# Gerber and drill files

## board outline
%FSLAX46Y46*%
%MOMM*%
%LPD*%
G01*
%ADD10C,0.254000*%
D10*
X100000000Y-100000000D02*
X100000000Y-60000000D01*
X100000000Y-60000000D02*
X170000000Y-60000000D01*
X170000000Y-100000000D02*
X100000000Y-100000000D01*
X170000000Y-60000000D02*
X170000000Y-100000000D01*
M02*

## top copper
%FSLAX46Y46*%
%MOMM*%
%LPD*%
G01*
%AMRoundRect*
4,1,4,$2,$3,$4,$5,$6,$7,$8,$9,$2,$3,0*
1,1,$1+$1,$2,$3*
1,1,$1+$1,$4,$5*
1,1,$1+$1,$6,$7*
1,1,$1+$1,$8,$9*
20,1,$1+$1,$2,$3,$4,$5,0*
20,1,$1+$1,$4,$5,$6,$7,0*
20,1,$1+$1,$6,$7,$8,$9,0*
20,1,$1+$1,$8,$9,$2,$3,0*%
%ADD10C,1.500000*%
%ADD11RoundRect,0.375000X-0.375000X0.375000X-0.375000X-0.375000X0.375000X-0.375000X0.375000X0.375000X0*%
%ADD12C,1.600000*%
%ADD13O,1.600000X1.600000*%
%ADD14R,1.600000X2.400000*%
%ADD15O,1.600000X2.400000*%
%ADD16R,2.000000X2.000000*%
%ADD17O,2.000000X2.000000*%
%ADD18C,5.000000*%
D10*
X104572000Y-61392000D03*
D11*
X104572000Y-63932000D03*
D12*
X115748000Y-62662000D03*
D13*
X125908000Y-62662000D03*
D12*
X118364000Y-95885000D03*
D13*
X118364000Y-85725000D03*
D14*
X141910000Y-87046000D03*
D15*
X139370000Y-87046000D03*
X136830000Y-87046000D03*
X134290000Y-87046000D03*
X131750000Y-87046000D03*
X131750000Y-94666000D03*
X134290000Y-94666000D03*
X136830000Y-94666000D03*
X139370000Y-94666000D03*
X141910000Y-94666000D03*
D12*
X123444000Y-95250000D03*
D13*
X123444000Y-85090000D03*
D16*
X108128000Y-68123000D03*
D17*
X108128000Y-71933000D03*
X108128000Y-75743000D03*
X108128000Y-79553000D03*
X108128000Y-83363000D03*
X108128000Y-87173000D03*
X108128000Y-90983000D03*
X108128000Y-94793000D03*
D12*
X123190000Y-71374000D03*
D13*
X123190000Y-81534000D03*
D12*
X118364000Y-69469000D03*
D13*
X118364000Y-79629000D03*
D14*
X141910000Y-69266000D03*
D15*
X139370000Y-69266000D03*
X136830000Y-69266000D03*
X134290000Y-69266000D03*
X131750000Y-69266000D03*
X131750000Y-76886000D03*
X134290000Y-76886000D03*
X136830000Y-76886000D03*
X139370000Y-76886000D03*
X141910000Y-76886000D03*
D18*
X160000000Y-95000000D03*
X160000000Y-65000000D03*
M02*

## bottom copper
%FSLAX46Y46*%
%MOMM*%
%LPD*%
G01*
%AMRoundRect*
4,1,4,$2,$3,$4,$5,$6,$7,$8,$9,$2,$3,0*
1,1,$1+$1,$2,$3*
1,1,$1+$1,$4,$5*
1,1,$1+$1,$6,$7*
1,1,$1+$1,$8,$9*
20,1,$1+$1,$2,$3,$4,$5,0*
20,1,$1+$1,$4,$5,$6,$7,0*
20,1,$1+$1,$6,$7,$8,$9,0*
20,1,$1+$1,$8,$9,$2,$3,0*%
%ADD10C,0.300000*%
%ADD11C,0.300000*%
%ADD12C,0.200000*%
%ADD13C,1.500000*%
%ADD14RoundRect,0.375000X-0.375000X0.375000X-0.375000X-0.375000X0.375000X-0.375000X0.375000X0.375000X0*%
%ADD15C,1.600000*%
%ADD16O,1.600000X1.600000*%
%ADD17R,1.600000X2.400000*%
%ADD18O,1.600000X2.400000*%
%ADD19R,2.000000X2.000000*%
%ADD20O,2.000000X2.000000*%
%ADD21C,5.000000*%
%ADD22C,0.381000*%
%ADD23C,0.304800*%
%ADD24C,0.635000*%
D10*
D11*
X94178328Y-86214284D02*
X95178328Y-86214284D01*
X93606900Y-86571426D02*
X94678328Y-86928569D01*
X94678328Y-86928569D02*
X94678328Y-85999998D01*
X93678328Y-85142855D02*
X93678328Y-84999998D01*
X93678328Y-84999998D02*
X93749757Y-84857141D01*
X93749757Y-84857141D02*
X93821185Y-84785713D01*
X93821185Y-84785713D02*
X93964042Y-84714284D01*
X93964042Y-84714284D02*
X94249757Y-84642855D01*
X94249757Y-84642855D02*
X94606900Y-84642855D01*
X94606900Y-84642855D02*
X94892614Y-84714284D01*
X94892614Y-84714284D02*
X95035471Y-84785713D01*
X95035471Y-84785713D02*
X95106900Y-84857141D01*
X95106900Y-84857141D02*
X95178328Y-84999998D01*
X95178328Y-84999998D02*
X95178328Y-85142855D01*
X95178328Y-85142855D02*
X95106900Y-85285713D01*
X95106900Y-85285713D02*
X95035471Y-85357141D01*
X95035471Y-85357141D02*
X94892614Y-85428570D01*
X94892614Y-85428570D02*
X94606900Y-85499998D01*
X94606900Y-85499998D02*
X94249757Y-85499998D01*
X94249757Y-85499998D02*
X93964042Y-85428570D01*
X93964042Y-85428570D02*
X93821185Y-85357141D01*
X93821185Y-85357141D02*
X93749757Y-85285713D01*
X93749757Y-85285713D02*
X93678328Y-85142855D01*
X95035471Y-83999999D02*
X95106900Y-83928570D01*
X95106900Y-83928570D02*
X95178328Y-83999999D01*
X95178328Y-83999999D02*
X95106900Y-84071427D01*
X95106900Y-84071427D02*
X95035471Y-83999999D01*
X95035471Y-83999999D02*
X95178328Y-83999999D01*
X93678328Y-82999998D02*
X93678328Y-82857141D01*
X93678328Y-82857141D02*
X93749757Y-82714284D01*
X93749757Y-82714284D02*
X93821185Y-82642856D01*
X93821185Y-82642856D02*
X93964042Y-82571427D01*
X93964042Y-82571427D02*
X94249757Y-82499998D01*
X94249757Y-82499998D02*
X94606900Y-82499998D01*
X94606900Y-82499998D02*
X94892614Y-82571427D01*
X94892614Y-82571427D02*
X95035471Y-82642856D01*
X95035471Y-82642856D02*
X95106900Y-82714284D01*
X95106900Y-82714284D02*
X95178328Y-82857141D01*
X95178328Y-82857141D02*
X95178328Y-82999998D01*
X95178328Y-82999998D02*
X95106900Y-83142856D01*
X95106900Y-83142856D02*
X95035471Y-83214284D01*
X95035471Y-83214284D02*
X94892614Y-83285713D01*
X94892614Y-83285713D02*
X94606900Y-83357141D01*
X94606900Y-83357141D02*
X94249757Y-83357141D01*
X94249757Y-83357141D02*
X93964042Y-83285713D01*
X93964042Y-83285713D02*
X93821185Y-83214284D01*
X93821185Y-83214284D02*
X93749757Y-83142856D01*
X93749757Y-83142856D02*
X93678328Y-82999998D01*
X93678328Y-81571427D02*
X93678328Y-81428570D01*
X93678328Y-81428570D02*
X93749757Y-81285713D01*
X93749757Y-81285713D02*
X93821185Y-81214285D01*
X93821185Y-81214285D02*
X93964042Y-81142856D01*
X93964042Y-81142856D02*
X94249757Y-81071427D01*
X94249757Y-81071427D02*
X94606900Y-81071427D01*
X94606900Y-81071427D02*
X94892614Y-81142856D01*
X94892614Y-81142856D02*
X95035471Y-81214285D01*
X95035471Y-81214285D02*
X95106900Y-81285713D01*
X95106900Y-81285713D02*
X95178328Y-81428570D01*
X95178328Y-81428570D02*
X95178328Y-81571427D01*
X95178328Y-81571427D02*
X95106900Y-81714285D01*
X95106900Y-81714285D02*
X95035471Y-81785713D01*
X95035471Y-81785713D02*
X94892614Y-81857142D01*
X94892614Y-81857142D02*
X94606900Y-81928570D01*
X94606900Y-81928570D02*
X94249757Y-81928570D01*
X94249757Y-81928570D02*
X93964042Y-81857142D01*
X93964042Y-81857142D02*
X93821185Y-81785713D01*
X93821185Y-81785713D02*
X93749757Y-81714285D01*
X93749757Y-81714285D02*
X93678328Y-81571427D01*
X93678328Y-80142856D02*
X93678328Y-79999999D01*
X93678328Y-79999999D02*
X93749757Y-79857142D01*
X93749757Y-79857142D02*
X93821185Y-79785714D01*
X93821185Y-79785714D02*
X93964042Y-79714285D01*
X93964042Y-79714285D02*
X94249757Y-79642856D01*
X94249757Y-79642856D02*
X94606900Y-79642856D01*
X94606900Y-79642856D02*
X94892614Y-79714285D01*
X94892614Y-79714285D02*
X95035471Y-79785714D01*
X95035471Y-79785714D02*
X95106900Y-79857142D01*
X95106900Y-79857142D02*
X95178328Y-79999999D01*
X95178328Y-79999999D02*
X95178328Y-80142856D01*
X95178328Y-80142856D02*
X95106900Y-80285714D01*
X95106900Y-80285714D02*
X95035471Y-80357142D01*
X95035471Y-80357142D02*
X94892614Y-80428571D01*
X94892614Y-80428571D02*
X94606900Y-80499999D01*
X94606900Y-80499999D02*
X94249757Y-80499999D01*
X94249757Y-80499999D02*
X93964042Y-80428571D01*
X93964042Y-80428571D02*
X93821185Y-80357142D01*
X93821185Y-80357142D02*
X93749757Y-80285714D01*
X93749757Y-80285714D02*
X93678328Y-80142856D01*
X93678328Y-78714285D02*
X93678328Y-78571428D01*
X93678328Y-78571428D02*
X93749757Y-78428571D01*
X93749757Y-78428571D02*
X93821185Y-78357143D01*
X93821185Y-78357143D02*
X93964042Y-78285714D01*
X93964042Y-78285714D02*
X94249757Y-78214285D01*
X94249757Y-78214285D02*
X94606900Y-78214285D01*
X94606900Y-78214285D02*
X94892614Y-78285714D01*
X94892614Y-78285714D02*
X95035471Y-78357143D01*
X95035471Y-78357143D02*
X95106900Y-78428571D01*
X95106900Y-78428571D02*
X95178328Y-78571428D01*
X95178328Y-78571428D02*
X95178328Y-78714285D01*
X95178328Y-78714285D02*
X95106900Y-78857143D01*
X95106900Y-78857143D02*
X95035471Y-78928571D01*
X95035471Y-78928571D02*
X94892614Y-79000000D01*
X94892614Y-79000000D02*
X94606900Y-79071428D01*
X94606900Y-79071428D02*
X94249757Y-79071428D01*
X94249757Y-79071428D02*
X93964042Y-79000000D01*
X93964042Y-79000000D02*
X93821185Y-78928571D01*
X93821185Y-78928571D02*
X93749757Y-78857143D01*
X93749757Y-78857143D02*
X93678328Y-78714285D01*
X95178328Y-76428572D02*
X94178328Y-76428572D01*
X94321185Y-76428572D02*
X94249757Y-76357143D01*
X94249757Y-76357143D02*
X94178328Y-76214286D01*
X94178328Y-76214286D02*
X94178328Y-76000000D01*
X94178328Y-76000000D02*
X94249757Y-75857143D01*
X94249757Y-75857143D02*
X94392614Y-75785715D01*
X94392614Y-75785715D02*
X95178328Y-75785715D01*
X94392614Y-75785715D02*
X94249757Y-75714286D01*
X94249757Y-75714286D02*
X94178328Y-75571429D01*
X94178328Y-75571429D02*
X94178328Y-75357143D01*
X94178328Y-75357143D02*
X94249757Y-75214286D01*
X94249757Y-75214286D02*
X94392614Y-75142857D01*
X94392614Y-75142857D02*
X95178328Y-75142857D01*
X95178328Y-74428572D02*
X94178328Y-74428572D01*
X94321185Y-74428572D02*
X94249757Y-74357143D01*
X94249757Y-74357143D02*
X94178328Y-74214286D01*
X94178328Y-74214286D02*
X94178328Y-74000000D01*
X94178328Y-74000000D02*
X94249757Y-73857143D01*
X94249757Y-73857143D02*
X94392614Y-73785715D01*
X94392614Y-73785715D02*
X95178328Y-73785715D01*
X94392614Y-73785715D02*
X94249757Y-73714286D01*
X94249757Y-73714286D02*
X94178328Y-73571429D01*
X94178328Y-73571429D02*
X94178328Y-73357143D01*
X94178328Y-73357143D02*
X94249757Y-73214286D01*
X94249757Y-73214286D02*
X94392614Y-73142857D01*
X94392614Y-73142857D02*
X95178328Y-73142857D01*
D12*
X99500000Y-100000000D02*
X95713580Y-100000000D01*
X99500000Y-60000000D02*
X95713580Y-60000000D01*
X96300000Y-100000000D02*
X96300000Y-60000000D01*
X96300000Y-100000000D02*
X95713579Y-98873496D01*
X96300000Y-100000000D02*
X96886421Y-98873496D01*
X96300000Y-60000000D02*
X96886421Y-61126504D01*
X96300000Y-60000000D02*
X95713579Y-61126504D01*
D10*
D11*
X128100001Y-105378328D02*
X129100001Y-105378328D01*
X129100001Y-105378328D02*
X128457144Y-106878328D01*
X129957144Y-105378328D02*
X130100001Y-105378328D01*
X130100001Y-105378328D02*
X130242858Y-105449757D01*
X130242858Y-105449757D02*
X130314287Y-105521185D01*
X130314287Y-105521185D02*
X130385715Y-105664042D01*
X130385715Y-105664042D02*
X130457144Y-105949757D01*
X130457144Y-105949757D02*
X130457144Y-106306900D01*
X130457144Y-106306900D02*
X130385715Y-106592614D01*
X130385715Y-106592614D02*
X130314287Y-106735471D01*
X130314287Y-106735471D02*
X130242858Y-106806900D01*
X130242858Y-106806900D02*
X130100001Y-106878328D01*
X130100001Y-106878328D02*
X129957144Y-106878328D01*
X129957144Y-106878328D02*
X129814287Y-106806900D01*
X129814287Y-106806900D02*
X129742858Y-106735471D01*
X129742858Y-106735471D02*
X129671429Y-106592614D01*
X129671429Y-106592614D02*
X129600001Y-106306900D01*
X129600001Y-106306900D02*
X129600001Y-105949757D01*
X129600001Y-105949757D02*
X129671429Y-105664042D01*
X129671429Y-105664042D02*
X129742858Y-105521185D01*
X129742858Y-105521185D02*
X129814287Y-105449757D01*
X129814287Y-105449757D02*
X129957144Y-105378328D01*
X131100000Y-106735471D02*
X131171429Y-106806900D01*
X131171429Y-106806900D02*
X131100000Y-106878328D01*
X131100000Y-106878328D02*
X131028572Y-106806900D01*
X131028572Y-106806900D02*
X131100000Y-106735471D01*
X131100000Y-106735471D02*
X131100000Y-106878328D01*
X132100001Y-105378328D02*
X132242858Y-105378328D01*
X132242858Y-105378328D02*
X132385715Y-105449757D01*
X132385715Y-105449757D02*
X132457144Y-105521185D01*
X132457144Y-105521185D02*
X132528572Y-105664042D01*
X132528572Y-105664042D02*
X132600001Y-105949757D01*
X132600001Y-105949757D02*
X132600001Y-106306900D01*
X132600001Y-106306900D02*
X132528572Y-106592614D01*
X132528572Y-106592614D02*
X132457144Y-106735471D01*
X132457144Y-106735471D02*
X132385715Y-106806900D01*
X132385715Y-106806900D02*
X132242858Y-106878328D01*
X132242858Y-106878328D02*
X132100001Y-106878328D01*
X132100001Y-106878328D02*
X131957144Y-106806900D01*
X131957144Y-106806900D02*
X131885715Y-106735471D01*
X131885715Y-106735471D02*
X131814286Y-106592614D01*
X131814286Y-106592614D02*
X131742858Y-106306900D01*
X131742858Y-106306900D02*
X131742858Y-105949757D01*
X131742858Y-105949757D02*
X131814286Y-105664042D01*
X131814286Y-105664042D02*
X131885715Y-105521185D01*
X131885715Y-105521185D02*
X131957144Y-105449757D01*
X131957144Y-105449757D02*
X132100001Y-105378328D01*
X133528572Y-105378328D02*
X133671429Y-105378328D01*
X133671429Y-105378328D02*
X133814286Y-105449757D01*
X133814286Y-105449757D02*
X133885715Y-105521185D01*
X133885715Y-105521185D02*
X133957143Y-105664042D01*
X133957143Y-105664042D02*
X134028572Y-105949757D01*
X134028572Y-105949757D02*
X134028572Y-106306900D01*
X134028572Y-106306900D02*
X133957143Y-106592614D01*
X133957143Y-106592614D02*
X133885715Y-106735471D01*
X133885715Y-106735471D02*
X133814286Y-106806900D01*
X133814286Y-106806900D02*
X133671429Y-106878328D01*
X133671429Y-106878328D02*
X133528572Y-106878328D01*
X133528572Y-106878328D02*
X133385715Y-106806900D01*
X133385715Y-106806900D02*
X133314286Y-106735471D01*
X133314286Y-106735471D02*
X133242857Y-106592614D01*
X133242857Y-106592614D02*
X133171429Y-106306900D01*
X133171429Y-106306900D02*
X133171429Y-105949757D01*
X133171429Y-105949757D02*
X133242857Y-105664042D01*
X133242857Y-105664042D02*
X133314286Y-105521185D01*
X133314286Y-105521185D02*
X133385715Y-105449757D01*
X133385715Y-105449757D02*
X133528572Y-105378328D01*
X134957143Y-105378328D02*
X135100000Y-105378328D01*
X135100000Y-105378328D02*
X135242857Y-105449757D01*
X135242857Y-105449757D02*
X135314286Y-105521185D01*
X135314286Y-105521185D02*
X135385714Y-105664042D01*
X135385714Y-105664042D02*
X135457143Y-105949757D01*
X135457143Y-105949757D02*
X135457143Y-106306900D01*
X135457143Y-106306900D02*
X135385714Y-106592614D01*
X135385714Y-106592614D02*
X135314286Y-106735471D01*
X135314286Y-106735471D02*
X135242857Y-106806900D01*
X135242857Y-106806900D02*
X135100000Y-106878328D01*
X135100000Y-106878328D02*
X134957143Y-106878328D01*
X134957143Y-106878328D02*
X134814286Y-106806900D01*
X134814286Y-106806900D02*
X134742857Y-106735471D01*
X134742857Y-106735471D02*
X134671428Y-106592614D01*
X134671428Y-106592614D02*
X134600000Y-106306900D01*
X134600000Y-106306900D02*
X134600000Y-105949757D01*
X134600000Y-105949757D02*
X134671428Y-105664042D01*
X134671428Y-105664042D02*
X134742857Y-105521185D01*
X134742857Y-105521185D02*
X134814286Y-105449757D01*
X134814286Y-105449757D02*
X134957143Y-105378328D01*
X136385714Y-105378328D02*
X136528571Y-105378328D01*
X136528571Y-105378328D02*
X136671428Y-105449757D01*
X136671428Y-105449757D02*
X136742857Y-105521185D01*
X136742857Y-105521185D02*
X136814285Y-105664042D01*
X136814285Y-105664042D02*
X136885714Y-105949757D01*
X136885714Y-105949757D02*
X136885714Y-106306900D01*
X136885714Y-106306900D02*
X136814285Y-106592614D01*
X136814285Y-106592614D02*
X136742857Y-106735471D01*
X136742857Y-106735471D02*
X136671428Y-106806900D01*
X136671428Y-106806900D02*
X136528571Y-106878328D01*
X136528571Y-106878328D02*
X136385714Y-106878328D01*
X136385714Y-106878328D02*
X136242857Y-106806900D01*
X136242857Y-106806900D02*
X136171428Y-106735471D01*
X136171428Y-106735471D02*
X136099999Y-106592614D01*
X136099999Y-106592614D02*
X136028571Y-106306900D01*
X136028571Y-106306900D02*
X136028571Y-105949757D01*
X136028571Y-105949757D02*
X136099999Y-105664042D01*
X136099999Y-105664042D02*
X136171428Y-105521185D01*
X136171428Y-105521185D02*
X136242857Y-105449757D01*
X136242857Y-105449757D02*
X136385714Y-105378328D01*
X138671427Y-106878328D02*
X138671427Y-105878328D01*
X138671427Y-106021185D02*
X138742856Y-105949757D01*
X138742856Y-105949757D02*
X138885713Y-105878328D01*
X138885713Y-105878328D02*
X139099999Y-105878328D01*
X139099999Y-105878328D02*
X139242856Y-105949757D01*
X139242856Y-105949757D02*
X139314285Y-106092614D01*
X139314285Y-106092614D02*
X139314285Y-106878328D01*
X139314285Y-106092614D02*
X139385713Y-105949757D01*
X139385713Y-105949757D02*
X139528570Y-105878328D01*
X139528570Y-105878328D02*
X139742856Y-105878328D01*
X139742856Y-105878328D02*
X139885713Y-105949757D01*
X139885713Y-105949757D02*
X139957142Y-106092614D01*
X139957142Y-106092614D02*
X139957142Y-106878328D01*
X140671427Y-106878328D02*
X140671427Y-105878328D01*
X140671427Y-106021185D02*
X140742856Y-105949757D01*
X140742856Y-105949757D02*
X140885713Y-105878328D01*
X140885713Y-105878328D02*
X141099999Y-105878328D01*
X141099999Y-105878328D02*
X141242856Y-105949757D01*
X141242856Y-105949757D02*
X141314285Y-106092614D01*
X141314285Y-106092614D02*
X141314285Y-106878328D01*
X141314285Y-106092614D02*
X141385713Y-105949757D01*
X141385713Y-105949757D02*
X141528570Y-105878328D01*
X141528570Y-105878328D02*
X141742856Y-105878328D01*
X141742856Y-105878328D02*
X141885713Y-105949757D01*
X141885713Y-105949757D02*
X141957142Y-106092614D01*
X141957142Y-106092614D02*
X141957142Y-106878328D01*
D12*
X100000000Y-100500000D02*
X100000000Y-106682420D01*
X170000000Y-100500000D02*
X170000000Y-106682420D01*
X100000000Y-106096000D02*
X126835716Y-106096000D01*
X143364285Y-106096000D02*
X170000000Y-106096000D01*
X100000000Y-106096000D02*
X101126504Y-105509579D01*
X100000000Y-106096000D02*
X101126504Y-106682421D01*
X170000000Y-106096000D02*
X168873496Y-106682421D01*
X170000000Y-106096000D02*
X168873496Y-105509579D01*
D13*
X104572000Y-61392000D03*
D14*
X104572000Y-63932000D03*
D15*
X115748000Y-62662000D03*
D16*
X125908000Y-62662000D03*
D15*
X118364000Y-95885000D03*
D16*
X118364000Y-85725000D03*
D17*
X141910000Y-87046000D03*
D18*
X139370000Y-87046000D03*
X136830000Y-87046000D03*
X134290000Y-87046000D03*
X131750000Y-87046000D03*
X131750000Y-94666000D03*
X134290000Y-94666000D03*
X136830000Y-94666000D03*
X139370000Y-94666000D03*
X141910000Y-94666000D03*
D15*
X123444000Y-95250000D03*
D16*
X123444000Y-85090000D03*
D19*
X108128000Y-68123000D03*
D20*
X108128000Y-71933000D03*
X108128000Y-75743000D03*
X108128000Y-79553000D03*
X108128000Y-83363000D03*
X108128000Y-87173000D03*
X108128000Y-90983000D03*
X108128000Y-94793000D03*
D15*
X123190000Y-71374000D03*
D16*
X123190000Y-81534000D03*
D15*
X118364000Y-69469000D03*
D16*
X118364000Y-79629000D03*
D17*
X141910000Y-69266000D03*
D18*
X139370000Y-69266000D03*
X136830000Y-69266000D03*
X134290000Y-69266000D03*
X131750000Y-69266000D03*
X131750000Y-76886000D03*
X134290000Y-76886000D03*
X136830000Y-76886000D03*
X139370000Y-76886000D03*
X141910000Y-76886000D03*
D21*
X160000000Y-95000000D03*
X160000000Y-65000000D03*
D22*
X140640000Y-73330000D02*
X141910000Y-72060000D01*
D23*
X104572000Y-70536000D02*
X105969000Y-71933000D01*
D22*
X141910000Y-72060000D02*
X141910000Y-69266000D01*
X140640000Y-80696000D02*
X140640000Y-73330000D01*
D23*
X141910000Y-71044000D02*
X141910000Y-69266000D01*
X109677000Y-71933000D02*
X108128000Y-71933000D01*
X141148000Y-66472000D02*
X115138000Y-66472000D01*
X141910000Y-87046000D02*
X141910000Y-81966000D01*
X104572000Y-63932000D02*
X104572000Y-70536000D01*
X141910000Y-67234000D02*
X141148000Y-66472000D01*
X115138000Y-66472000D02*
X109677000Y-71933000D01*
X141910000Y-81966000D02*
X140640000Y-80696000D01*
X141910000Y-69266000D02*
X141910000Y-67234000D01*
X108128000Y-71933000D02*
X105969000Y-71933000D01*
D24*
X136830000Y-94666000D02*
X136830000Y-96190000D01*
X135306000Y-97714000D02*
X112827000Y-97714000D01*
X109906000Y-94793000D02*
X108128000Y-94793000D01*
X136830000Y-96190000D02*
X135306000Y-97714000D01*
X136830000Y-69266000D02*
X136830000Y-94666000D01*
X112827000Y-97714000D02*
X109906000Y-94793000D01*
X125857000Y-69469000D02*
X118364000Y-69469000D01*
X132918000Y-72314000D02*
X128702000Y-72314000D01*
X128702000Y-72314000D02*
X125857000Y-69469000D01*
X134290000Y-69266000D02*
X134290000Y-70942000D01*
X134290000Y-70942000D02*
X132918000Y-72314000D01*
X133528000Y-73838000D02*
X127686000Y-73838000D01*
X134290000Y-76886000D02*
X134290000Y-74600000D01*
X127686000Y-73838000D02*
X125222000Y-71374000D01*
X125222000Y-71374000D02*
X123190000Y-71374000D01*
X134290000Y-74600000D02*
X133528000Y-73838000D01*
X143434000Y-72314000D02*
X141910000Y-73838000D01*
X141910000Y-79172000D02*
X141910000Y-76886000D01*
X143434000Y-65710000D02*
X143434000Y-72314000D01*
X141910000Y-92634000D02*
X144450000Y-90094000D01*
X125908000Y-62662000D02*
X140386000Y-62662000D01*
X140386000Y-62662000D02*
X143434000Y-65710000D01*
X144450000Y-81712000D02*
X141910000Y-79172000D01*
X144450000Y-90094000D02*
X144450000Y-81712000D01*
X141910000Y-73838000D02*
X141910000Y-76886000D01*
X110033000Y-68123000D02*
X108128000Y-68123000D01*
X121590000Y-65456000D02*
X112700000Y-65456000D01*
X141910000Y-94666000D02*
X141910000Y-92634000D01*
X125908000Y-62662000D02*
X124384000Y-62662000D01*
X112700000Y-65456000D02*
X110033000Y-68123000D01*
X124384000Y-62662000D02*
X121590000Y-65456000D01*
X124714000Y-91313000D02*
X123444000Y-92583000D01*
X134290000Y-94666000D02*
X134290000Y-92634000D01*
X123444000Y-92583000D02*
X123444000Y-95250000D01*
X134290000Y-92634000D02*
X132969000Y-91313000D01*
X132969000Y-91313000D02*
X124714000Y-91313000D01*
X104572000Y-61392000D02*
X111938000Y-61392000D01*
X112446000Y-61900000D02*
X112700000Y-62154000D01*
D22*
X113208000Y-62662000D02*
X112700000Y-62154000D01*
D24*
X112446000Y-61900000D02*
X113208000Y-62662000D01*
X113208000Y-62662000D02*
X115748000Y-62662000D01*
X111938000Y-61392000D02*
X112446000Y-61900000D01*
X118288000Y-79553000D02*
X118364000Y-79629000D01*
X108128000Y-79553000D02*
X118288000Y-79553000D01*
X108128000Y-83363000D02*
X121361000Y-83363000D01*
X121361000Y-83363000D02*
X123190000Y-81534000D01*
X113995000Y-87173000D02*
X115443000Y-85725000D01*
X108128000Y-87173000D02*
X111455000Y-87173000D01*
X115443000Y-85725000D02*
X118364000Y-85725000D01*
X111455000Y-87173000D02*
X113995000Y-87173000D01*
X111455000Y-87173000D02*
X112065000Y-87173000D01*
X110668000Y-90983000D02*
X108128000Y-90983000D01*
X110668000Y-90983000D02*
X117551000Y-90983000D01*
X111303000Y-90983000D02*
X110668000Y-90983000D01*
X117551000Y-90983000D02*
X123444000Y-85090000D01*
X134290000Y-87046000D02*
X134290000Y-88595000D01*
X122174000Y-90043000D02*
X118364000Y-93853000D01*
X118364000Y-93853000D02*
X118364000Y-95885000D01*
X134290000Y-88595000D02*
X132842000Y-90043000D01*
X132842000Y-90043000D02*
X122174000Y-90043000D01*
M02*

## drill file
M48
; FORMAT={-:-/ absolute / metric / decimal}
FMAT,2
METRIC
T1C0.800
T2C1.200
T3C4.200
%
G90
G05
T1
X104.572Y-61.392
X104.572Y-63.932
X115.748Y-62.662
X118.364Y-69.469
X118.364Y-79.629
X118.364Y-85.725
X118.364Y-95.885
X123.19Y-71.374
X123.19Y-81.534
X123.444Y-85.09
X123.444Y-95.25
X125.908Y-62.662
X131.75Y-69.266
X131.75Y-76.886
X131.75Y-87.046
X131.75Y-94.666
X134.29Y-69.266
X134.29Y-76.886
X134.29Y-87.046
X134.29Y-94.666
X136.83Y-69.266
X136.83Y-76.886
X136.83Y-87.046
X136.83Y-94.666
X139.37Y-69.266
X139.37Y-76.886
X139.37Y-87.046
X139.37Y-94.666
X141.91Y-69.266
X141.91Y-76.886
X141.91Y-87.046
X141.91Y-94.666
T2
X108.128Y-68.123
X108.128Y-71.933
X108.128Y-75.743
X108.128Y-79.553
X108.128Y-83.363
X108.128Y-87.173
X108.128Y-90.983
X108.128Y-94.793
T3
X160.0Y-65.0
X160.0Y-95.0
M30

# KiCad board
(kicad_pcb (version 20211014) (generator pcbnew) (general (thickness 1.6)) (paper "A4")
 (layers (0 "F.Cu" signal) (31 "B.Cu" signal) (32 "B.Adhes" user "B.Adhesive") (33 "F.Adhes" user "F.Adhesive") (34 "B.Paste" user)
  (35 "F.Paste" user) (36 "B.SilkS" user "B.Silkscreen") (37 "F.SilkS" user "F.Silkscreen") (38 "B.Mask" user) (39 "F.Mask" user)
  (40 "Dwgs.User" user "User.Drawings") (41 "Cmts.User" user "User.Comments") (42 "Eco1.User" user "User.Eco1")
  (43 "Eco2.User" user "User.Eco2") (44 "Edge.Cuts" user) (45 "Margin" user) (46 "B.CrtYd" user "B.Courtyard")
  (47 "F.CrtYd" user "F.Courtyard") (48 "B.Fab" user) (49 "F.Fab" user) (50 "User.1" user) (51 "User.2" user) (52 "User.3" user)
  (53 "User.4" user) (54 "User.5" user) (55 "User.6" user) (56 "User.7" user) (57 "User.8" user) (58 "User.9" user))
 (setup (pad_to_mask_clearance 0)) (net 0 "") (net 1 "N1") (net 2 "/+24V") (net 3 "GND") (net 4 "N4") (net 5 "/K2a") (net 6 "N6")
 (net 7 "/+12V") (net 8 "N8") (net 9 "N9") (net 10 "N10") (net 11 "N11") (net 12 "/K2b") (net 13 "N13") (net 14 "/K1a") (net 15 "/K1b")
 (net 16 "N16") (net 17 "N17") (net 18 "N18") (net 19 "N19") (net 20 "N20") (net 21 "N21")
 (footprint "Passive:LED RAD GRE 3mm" (layer "F.Cu") (at 104.572 62.662 -90)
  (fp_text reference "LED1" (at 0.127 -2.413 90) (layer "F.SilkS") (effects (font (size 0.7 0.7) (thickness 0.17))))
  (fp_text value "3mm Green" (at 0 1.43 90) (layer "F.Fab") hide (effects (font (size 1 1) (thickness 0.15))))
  (pad "1" thru_hole circle (at -1.27 0 270) (size 1.5 1.5) (drill 0.8) (layers *.Cu *.Mask) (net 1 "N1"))
  (pad "2" thru_hole roundrect (at 1.27 0 270) (size 1.5 1.5) (drill 0.8) (layers *.Cu *.Mask) (roundrect_rratio 0.25) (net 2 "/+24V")))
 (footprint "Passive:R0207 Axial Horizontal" (layer "F.Cu") (at 120.828 62.662)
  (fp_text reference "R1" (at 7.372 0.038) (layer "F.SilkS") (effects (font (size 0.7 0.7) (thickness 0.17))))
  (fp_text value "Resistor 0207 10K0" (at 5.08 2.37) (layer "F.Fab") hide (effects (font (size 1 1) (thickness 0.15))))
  (pad "1" thru_hole circle (at -5.08 0) (size 1.6 1.6) (drill 0.8) (layers *.Cu *.Mask) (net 1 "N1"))
  (pad "2" thru_hole oval (at 5.08 0) (size 1.6 1.6) (drill 0.8) (layers *.Cu *.Mask) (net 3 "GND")))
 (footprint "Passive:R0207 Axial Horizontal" (layer "F.Cu") (at 118.364 90.805 90)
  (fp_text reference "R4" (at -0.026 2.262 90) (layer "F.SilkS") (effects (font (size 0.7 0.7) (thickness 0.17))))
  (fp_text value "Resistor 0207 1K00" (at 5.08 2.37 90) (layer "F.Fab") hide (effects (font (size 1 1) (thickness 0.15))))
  (pad "1" thru_hole circle (at -5.08 0 90) (size 1.6 1.6) (drill 0.8) (layers *.Cu *.Mask) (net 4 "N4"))
  (pad "2" thru_hole oval (at 5.08 0 90) (size 1.6 1.6) (drill 0.8) (layers *.Cu *.Mask) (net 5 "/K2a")))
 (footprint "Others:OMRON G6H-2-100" (layer "F.Cu") (at 136.83 90.856 -90)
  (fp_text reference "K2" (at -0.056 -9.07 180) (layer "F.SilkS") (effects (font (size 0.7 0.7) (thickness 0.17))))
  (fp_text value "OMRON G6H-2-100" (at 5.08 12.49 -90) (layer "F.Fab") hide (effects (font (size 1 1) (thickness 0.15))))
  (pad "1" thru_hole rect (at -3.81 -5.08 270) (size 2.4 1.6) (drill 0.8) (layers *.Cu *.Mask) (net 2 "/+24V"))
  (pad "2" thru_hole oval (at -3.81 -2.54 270) (size 2.4 1.6) (drill 0.8) (layers *.Cu *.Mask) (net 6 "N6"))
  (pad "3" thru_hole oval (at -3.81 0 270) (size 2.4 1.6) (drill 0.8) (layers *.Cu *.Mask) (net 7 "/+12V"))
  (pad "4" thru_hole oval (at -3.81 2.54 270) (size 2.4 1.6) (drill 0.8) (layers *.Cu *.Mask) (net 4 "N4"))
  (pad "5" thru_hole oval (at -3.81 5.08 270) (size 2.4 1.6) (drill 0.8) (layers *.Cu *.Mask) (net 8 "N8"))
  (pad "6" thru_hole oval (at 3.81 5.08 270) (size 2.4 1.6) (drill 0.8) (layers *.Cu *.Mask) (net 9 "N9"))
  (pad "7" thru_hole oval (at 3.81 2.54 270) (size 2.4 1.6) (drill 0.8) (layers *.Cu *.Mask) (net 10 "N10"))
  (pad "8" thru_hole oval (at 3.81 0 270) (size 2.4 1.6) (drill 0.8) (layers *.Cu *.Mask) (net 7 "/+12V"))
  (pad "9" thru_hole oval (at 3.81 -2.54 270) (size 2.4 1.6) (drill 0.8) (layers *.Cu *.Mask) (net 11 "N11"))
  (pad "10" thru_hole oval (at 3.81 -5.08 270) (size 2.4 1.6) (drill 0.8) (layers *.Cu *.Mask) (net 3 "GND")))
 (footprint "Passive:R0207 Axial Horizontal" (layer "F.Cu") (at 123.444 90.17 90)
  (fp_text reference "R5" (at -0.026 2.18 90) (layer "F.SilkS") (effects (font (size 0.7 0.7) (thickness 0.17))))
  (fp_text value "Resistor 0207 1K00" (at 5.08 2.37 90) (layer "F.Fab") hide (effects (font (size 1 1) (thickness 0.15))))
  (pad "1" thru_hole circle (at -5.08 0 90) (size 1.6 1.6) (drill 0.8) (layers *.Cu *.Mask) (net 10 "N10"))
  (pad "2" thru_hole oval (at 5.08 0 90) (size 1.6 1.6) (drill 0.8) (layers *.Cu *.Mask) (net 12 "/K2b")))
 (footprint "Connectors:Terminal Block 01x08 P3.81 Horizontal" (layer "F.Cu") (at 108.128 81.458 -90)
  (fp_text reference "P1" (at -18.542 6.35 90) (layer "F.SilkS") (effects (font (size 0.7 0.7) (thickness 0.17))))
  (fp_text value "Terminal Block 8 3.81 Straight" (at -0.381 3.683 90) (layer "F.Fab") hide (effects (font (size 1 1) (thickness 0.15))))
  (pad "1" thru_hole rect (at -13.335 0) (size 2 2) (drill 1.2) (layers *.Cu *.Mask) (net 3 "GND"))
  (pad "2" thru_hole oval (at -9.525 0) (size 2 2) (drill 1.2) (layers *.Cu *.Mask) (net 2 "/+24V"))
  (pad "3" thru_hole oval (at -5.715 0) (size 2 2) (drill 1.2) (layers *.Cu *.Mask) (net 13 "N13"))
  (pad "4" thru_hole oval (at -1.905 0) (size 2 2) (drill 1.2) (layers *.Cu *.Mask) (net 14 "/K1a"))
  (pad "5" thru_hole oval (at 1.905 0) (size 2 2) (drill 1.2) (layers *.Cu *.Mask) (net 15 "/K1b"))
  (pad "6" thru_hole oval (at 5.715 0) (size 2 2) (drill 1.2) (layers *.Cu *.Mask) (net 5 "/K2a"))
  (pad "7" thru_hole oval (at 9.525 0) (size 2 2) (drill 1.2) (layers *.Cu *.Mask) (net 12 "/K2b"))
  (pad "8" thru_hole oval (at 13.335 0) (size 2 2) (drill 1.2) (layers *.Cu *.Mask) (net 7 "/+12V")))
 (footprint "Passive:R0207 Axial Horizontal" (layer "F.Cu") (at 123.19 76.454 -90)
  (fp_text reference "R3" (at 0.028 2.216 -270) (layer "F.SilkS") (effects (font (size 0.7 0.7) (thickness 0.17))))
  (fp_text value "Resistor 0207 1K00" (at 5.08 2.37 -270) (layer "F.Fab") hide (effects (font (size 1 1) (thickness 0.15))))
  (pad "1" thru_hole circle (at -5.08 0 270) (size 1.6 1.6) (drill 0.8) (layers *.Cu *.Mask) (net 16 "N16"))
  (pad "2" thru_hole oval (at 5.08 0 270) (size 1.6 1.6) (drill 0.8) (layers *.Cu *.Mask) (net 15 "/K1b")))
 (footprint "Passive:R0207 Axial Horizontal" (layer "F.Cu") (at 118.364 74.549 -90)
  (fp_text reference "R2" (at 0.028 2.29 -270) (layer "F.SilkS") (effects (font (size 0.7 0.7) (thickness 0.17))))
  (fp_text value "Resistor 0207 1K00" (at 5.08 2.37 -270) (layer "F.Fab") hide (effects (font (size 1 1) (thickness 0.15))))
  (pad "1" thru_hole circle (at -5.08 0 270) (size 1.6 1.6) (drill 0.8) (layers *.Cu *.Mask) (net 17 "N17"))
  (pad "2" thru_hole oval (at 5.08 0 270) (size 1.6 1.6) (drill 0.8) (layers *.Cu *.Mask) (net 14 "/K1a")))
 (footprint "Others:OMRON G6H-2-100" (layer "F.Cu") (at 136.83 73.076 -90)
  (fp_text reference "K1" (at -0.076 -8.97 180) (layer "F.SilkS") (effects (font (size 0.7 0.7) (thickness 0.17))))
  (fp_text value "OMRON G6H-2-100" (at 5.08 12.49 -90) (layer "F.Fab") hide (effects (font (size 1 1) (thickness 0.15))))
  (pad "1" thru_hole rect (at -3.81 -5.08 270) (size 2.4 1.6) (drill 0.8) (layers *.Cu *.Mask) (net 2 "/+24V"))
  (pad "2" thru_hole oval (at -3.81 -2.54 270) (size 2.4 1.6) (drill 0.8) (layers *.Cu *.Mask) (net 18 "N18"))
  (pad "3" thru_hole oval (at -3.81 0 270) (size 2.4 1.6) (drill 0.8) (layers *.Cu *.Mask) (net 7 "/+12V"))
  (pad "4" thru_hole oval (at -3.81 2.54 270) (size 2.4 1.6) (drill 0.8) (layers *.Cu *.Mask) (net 17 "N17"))
  (pad "5" thru_hole oval (at -3.81 5.08 270) (size 2.4 1.6) (drill 0.8) (layers *.Cu *.Mask) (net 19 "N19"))
  (pad "6" thru_hole oval (at 3.81 5.08 270) (size 2.4 1.6) (drill 0.8) (layers *.Cu *.Mask) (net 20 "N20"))
  (pad "7" thru_hole oval (at 3.81 2.54 270) (size 2.4 1.6) (drill 0.8) (layers *.Cu *.Mask) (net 16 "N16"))
  (pad "8" thru_hole oval (at 3.81 0 270) (size 2.4 1.6) (drill 0.8) (layers *.Cu *.Mask) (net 7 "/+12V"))
  (pad "9" thru_hole oval (at 3.81 -2.54 270) (size 2.4 1.6) (drill 0.8) (layers *.Cu *.Mask) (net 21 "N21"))
  (pad "10" thru_hole oval (at 3.81 -5.08 270) (size 2.4 1.6) (drill 0.8) (layers *.Cu *.Mask) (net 3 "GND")))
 (gr_line (start 100 100) (end 100 60) (layer "Edge.Cuts") (width 0.254))
 (gr_line (start 100 60) (end 170 60) (layer "Edge.Cuts") (width 0.254))
 (gr_line (start 170 100) (end 100 100) (layer "Edge.Cuts") (width 0.254))
 (gr_line (start 170 60) (end 170 100) (layer "Edge.Cuts") (width 0.254))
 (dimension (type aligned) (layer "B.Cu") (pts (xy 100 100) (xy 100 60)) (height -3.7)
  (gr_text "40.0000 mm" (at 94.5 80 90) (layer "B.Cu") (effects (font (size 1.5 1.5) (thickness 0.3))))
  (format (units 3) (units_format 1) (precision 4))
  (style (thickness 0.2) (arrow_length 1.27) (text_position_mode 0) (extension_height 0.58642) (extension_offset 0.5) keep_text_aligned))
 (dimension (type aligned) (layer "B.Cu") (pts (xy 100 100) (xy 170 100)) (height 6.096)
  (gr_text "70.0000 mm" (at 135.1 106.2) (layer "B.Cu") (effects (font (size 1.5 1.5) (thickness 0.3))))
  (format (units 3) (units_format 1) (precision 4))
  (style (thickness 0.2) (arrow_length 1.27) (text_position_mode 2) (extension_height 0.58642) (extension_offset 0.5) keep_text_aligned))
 (via (at 160 95) (size 5) (drill 4.2) (layers "F.Cu" "B.Cu") (free) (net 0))
 (via (at 160 65) (size 5) (drill 4.2) (layers "F.Cu" "B.Cu") (free) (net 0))
 (segment (start 140.64 73.33) (end 141.91 72.06) (width 0.381) (layer "B.Cu") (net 2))
 (segment (start 104.572 70.536) (end 105.969 71.933) (width 0.3048) (layer "B.Cu") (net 2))
 (segment (start 141.91 72.06) (end 141.91 69.266) (width 0.381) (layer "B.Cu") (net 2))
 (segment (start 140.64 80.696) (end 140.64 73.33) (width 0.381) (layer "B.Cu") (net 2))
 (segment (start 141.91 71.044) (end 141.91 69.266) (width 0.3048) (layer "B.Cu") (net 2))
 (segment (start 109.677 71.933) (end 108.128 71.933) (width 0.3048) (layer "B.Cu") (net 2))
 (segment (start 141.148 66.472) (end 115.138 66.472) (width 0.3048) (layer "B.Cu") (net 2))
 (segment (start 141.91 87.046) (end 141.91 81.966) (width 0.3048) (layer "B.Cu") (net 2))
 (segment (start 104.572 63.932) (end 104.572 70.536) (width 0.3048) (layer "B.Cu") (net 2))
 (segment (start 141.91 67.234) (end 141.148 66.472) (width 0.3048) (layer "B.Cu") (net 2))
 (segment (start 115.138 66.472) (end 109.677 71.933) (width 0.3048) (layer "B.Cu") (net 2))
 (segment (start 141.91 81.966) (end 140.64 80.696) (width 0.3048) (layer "B.Cu") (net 2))
 (segment (start 141.91 69.266) (end 141.91 67.234) (width 0.3048) (layer "B.Cu") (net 2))
 (segment (start 108.128 71.933) (end 105.969 71.933) (width 0.3048) (layer "B.Cu") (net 2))
 (segment (start 136.83 94.666) (end 136.83 96.19) (width 0.635) (layer "B.Cu") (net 7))
 (segment (start 135.306 97.714) (end 112.827 97.714) (width 0.635) (layer "B.Cu") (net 7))
 (segment (start 109.906 94.793) (end 108.128 94.793) (width 0.635) (layer "B.Cu") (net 7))
 (segment (start 136.83 96.19) (end 135.306 97.714) (width 0.635) (layer "B.Cu") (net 7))
 (segment (start 136.83 69.266) (end 136.83 94.666) (width 0.635) (layer "B.Cu") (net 7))
 (segment (start 112.827 97.714) (end 109.906 94.793) (width 0.635) (layer "B.Cu") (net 7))
 (segment (start 125.857 69.469) (end 118.364 69.469) (width 0.635) (layer "B.Cu") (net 17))
 (segment (start 132.918 72.314) (end 128.702 72.314) (width 0.635) (layer "B.Cu") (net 17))
 (segment (start 128.702 72.314) (end 125.857 69.469) (width 0.635) (layer "B.Cu") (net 17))
 (segment (start 134.29 69.266) (end 134.29 70.942) (width 0.635) (layer "B.Cu") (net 17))
 (segment (start 134.29 70.942) (end 132.918 72.314) (width 0.635) (layer "B.Cu") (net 17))
 (segment (start 133.528 73.838) (end 127.686 73.838) (width 0.635) (layer "B.Cu") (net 16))
 (segment (start 134.29 76.886) (end 134.29 74.6) (width 0.635) (layer "B.Cu") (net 16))
 (segment (start 127.686 73.838) (end 125.222 71.374) (width 0.635) (layer "B.Cu") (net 16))
 (segment (start 125.222 71.374) (end 123.19 71.374) (width 0.635) (layer "B.Cu") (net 16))
 (segment (start 134.29 74.6) (end 133.528 73.838) (width 0.635) (layer "B.Cu") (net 16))
 (segment (start 143.434 72.314) (end 141.91 73.838) (width 0.635) (layer "B.Cu") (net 3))
 (segment (start 141.91 79.172) (end 141.91 76.886) (width 0.635) (layer "B.Cu") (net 3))
 (segment (start 143.434 65.71) (end 143.434 72.314) (width 0.635) (layer "B.Cu") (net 3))
 (segment (start 141.91 92.634) (end 144.45 90.094) (width 0.635) (layer "B.Cu") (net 3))
 (segment (start 125.908 62.662) (end 140.386 62.662) (width 0.635) (layer "B.Cu") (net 3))
 (segment (start 140.386 62.662) (end 143.434 65.71) (width 0.635) (layer "B.Cu") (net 3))
 (segment (start 144.45 81.712) (end 141.91 79.172) (width 0.635) (layer "B.Cu") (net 3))
 (segment (start 144.45 90.094) (end 144.45 81.712) (width 0.635) (layer "B.Cu") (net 3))
 (segment (start 141.91 73.838) (end 141.91 76.886) (width 0.635) (layer "B.Cu") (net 3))
 (segment (start 110.033 68.123) (end 108.128 68.123) (width 0.635) (layer "B.Cu") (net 3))
 (segment (start 121.59 65.456) (end 112.7 65.456) (width 0.635) (layer "B.Cu") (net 3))
 (segment (start 141.91 94.666) (end 141.91 92.634) (width 0.635) (layer "B.Cu") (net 3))
 (segment (start 125.908 62.662) (end 124.384 62.662) (width 0.635) (layer "B.Cu") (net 3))
 (segment (start 112.7 65.456) (end 110.033 68.123) (width 0.635) (layer "B.Cu") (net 3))
 (segment (start 124.384 62.662) (end 121.59 65.456) (width 0.635) (layer "B.Cu") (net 3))
 (segment (start 124.714 91.313) (end 123.444 92.583) (width 0.635) (layer "B.Cu") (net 10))
 (segment (start 134.29 94.666) (end 134.29 92.634) (width 0.635) (layer "B.Cu") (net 10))
 (segment (start 123.444 92.583) (end 123.444 95.25) (width 0.635) (layer "B.Cu") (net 10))
 (segment (start 134.29 92.634) (end 132.969 91.313) (width 0.635) (layer "B.Cu") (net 10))
 (segment (start 132.969 91.313) (end 124.714 91.313) (width 0.635) (layer "B.Cu") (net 10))
 (segment (start 104.572 61.392) (end 111.938 61.392) (width 0.635) (layer "B.Cu") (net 1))
 (segment (start 112.446 61.9) (end 112.7 62.154) (width 0.635) (layer "B.Cu") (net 1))
 (segment (start 113.208 62.662) (end 112.7 62.154) (width 0.381) (layer "B.Cu") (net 1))
 (segment (start 112.446 61.9) (end 113.208 62.662) (width 0.635) (layer "B.Cu") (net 1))
 (segment (start 113.208 62.662) (end 115.748 62.662) (width 0.635) (layer "B.Cu") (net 1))
 (segment (start 111.938 61.392) (end 112.446 61.9) (width 0.635) (layer "B.Cu") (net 1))
 (segment (start 118.288 79.553) (end 118.364 79.629) (width 0.635) (layer "B.Cu") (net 14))
 (segment (start 108.128 79.553) (end 118.288 79.553) (width 0.635) (layer "B.Cu") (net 14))
 (segment (start 108.128 83.363) (end 121.361 83.363) (width 0.635) (layer "B.Cu") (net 15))
 (segment (start 121.361 83.363) (end 123.19 81.534) (width 0.635) (layer "B.Cu") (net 15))
 (segment (start 113.995 87.173) (end 115.443 85.725) (width 0.635) (layer "B.Cu") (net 5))
 (segment (start 108.128 87.173) (end 111.455 87.173) (width 0.635) (layer "B.Cu") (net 5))
 (segment (start 115.443 85.725) (end 118.364 85.725) (width 0.635) (layer "B.Cu") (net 5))
 (segment (start 111.455 87.173) (end 113.995 87.173) (width 0.635) (layer "B.Cu") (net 5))
 (segment (start 111.455 87.173) (end 112.065 87.173) (width 0.635) (layer "B.Cu") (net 5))
 (segment (start 110.668 90.983) (end 108.128 90.983) (width 0.635) (layer "B.Cu") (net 12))
 (segment (start 110.668 90.983) (end 117.551 90.983) (width 0.635) (layer "B.Cu") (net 12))
 (segment (start 111.303 90.983) (end 110.668 90.983) (width 0.635) (layer "B.Cu") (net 12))
 (segment (start 117.551 90.983) (end 123.444 85.09) (width 0.635) (layer "B.Cu") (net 12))
 (segment (start 134.29 87.046) (end 134.29 88.595) (width 0.635) (layer "B.Cu") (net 4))
 (segment (start 122.174 90.043) (end 118.364 93.853) (width 0.635) (layer "B.Cu") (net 4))
 (segment (start 118.364 93.853) (end 118.364 95.885) (width 0.635) (layer "B.Cu") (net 4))
 (segment (start 134.29 88.595) (end 132.842 90.043) (width 0.635) (layer "B.Cu") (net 4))
 (segment (start 132.842 90.043) (end 122.174 90.043) (width 0.635) (layer "B.Cu") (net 4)))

